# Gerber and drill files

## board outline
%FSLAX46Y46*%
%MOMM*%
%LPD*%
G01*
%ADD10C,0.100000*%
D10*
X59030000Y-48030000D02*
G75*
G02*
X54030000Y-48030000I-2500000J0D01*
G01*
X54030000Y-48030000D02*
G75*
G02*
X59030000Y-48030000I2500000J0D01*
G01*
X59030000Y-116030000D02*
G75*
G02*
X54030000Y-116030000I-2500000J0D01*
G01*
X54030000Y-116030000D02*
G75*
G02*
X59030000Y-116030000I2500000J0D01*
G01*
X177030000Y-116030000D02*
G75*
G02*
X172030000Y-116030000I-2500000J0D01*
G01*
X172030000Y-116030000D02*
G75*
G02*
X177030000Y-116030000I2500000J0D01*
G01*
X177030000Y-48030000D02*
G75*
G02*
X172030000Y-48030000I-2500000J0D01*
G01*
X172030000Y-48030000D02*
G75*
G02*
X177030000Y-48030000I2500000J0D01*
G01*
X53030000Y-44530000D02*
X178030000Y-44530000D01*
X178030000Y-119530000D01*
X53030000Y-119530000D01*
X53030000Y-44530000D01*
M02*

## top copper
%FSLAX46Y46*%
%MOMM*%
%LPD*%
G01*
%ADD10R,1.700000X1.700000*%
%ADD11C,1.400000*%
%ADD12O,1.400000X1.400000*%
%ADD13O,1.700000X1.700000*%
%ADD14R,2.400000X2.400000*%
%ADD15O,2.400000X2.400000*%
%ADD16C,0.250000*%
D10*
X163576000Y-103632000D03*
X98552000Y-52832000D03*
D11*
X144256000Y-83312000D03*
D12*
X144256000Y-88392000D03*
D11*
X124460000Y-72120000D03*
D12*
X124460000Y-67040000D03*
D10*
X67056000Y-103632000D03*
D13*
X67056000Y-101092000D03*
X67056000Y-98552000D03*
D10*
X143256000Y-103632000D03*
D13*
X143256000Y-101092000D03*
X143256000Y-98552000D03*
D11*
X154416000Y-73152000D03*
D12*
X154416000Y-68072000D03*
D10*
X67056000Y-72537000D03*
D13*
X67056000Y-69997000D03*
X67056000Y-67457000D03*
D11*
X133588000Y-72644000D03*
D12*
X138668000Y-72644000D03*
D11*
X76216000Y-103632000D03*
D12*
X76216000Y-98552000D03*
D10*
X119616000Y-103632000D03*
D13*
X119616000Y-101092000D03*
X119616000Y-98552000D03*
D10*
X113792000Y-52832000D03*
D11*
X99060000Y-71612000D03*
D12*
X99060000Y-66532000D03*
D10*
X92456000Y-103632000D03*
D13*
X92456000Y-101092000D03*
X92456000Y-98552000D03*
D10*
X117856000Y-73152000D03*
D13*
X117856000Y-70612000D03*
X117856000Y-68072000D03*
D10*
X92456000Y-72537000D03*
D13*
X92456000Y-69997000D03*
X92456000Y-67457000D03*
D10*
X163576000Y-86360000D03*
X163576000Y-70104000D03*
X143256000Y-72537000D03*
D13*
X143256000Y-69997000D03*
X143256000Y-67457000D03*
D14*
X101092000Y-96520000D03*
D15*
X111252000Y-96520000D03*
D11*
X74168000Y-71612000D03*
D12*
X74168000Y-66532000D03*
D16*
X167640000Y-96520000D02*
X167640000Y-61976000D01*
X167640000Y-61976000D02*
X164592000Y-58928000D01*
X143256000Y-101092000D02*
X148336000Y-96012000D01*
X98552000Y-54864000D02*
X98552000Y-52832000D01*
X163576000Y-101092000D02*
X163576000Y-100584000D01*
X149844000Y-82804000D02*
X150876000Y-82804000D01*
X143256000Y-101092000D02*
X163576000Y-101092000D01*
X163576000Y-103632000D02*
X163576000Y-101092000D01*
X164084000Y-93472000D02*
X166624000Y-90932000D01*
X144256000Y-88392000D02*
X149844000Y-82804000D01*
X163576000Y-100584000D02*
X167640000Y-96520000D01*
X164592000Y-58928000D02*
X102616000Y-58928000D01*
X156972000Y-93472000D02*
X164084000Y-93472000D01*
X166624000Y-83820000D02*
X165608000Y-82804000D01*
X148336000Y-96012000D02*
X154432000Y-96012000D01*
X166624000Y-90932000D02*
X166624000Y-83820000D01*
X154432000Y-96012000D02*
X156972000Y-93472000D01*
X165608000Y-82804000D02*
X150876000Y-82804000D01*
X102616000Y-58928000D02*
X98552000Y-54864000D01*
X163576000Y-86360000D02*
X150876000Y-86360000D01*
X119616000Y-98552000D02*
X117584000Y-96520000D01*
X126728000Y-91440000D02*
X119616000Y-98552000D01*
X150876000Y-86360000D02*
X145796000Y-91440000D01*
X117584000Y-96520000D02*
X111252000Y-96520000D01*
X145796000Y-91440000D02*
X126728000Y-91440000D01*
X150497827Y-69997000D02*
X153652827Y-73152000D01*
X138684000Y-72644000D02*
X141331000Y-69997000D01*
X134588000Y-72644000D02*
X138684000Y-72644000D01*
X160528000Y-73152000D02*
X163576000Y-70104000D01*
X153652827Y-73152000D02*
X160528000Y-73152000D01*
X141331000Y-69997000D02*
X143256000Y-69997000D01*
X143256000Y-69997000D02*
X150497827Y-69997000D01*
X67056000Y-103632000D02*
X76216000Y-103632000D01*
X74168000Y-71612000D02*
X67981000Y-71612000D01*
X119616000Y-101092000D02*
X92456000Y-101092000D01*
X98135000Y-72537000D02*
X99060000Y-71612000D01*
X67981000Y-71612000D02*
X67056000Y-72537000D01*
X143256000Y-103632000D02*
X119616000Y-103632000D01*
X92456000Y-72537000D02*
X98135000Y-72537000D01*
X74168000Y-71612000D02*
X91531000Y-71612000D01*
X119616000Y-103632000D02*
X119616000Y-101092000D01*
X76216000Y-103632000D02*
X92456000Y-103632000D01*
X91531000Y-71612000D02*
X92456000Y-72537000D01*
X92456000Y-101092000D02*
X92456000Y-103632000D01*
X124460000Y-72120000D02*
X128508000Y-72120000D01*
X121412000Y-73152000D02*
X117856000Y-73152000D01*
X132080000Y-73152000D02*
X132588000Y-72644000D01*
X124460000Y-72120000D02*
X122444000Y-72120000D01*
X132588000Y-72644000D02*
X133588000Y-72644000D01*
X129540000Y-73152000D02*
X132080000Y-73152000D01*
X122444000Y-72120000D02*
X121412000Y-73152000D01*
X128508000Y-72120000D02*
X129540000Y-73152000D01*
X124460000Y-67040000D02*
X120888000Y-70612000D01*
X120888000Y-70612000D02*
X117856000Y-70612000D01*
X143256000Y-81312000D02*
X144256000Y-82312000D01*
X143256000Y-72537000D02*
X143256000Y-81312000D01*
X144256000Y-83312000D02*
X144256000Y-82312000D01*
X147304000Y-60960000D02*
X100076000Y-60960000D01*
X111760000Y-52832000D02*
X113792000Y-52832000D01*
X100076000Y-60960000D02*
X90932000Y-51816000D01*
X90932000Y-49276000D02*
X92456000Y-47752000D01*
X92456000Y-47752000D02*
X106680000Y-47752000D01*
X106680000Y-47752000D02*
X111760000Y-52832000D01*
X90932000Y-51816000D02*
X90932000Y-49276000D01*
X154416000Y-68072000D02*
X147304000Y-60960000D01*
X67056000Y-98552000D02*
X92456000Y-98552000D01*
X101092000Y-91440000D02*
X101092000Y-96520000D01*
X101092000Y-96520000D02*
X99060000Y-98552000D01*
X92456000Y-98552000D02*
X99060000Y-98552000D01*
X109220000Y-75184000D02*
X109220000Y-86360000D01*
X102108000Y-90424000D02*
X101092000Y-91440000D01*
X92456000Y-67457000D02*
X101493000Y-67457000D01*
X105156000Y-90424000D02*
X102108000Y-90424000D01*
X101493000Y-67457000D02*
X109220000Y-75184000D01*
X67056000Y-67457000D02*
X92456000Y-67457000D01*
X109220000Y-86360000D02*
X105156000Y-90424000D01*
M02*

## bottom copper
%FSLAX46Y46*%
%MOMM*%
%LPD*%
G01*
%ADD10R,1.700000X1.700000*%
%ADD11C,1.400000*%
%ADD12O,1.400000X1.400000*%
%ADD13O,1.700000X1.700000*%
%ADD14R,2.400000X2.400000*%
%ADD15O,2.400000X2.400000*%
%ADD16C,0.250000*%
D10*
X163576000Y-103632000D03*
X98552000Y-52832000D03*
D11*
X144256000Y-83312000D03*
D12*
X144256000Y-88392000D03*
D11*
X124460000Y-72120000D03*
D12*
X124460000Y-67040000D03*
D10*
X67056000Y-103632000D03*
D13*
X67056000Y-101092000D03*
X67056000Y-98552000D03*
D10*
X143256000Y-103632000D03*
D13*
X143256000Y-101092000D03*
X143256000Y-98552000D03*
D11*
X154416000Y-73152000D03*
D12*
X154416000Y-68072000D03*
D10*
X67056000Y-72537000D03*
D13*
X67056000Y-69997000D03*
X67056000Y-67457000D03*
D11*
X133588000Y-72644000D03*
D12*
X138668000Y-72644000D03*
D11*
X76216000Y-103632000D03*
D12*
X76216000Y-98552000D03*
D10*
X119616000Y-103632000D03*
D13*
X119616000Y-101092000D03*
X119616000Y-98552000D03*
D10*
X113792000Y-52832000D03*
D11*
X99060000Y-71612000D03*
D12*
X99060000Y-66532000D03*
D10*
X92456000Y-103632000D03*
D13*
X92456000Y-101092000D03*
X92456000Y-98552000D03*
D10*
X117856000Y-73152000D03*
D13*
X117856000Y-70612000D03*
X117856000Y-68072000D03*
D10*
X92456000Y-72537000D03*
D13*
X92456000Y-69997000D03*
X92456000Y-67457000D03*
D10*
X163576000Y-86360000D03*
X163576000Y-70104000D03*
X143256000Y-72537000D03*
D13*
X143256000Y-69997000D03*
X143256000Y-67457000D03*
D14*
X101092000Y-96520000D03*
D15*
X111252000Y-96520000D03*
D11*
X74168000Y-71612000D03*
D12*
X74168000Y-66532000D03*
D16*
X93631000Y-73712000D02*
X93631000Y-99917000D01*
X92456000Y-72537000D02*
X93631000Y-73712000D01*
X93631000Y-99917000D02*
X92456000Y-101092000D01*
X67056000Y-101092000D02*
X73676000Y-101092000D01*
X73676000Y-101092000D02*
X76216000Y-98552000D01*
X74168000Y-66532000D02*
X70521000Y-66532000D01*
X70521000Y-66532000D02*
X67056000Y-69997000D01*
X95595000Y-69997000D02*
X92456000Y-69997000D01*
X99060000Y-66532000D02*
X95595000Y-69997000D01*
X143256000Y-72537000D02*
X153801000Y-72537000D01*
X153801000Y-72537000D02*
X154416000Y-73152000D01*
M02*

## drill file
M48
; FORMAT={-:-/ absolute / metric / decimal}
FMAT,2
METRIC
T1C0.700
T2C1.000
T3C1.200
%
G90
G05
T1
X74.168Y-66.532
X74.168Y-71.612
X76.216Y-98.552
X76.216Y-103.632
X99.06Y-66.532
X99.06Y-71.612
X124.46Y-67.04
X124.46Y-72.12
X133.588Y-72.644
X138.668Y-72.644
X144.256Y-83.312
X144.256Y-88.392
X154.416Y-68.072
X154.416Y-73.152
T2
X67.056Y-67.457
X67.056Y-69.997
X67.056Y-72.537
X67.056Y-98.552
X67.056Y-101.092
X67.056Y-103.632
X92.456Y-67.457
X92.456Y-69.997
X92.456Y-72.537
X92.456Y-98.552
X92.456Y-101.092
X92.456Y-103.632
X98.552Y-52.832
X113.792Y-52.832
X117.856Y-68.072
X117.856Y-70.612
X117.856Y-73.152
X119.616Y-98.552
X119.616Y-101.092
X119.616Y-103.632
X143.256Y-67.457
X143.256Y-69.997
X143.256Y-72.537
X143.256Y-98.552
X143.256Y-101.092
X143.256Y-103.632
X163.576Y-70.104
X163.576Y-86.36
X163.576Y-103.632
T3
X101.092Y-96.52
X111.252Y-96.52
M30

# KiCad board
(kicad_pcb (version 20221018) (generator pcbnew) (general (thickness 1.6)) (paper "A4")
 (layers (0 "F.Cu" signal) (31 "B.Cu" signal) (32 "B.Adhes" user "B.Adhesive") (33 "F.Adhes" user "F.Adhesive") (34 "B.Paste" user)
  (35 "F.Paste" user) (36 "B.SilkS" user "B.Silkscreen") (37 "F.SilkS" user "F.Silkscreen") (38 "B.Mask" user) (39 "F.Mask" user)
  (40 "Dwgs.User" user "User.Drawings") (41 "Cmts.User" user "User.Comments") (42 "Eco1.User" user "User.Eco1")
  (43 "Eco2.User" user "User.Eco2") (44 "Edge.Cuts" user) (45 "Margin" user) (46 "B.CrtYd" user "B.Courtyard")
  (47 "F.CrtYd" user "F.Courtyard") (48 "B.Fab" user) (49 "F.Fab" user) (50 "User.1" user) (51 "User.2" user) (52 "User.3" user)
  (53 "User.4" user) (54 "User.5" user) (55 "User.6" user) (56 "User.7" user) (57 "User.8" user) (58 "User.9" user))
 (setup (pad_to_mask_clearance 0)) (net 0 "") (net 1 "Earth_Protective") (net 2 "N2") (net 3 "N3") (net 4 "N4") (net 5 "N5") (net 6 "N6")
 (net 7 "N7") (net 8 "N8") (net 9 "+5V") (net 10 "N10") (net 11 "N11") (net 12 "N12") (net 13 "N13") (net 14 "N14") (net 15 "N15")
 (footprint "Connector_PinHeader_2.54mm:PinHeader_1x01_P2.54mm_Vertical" (layer "F.Cu") (at 163.576 103.632 180)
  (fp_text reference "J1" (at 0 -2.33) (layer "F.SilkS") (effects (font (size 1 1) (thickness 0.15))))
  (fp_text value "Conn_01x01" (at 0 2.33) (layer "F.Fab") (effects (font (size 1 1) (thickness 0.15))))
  (pad "1" thru_hole rect (at 0 0 180) (size 1.7 1.7) (drill 1) (layers "*.Cu" "*.Mask") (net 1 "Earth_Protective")))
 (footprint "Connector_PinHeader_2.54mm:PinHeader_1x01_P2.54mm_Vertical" (layer "F.Cu") (at 98.552 52.832 180)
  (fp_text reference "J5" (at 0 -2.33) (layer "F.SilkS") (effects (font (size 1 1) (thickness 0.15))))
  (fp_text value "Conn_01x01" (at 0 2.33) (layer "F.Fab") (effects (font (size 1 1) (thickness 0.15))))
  (pad "1" thru_hole rect (at 0 0 180) (size 1.7 1.7) (drill 1) (layers "*.Cu" "*.Mask") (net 1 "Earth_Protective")))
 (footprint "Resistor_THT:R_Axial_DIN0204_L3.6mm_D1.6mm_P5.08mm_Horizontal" (layer "F.Cu") (at 144.256 83.312 -90)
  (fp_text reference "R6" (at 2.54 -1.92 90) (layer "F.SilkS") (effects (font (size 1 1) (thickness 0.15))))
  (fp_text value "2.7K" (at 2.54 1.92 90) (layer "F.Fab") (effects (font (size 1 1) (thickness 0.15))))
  (pad "1" thru_hole circle (at 0 0 270) (size 1.4 1.4) (drill 0.7) (layers "*.Cu" "*.Mask") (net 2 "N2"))
  (pad "2" thru_hole oval (at 5.08 0 270) (size 1.4 1.4) (drill 0.7) (layers "*.Cu" "*.Mask") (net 1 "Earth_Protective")))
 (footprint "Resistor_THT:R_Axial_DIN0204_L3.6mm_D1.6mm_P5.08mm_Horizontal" (layer "F.Cu") (at 124.46 72.12 90)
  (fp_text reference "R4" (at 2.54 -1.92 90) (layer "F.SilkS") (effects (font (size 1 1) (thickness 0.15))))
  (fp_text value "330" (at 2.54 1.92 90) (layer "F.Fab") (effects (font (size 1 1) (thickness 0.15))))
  (pad "1" thru_hole circle (at 0 0 90) (size 1.4 1.4) (drill 0.7) (layers "*.Cu" "*.Mask") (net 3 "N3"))
  (pad "2" thru_hole oval (at 5.08 0 90) (size 1.4 1.4) (drill 0.7) (layers "*.Cu" "*.Mask") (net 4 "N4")))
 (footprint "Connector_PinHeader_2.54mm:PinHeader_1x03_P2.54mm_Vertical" (layer "F.Cu") (at 67.056 103.632 180)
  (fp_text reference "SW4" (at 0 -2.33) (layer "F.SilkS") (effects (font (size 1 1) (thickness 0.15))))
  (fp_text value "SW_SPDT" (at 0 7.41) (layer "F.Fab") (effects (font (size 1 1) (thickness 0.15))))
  (pad "1" thru_hole rect (at 0 0 180) (size 1.7 1.7) (drill 1) (layers "*.Cu" "*.Mask") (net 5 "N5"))
  (pad "2" thru_hole oval (at 0 2.54 180) (size 1.7 1.7) (drill 1) (layers "*.Cu" "*.Mask") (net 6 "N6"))
  (pad "3" thru_hole oval (at 0 5.08 180) (size 1.7 1.7) (drill 1) (layers "*.Cu" "*.Mask") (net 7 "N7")))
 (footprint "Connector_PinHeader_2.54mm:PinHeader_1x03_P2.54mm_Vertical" (layer "F.Cu") (at 143.256 103.632 180)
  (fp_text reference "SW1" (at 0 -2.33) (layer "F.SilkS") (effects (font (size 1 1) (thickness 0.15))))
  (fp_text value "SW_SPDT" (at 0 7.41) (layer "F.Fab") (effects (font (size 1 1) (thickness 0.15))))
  (pad "1" thru_hole rect (at 0 0 180) (size 1.7 1.7) (drill 1) (layers "*.Cu" "*.Mask") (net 5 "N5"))
  (pad "2" thru_hole oval (at 0 2.54 180) (size 1.7 1.7) (drill 1) (layers "*.Cu" "*.Mask") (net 1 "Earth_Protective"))
  (pad "3" thru_hole oval (at 0 5.08 180) (size 1.7 1.7) (drill 1) (layers "*.Cu" "*.Mask") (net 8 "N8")))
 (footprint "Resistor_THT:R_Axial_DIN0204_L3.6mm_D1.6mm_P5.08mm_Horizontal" (layer "F.Cu") (at 154.416 73.152 90)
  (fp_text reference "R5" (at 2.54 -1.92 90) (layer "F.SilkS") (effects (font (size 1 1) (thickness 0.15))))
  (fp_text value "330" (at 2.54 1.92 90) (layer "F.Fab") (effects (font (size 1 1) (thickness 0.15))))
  (pad "1" thru_hole circle (at 0 0 90) (size 1.4 1.4) (drill 0.7) (layers "*.Cu" "*.Mask") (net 2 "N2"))
  (pad "2" thru_hole oval (at 5.08 0 90) (size 1.4 1.4) (drill 0.7) (layers "*.Cu" "*.Mask") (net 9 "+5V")))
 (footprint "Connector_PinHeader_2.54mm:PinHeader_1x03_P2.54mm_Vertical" (layer "F.Cu") (at 67.056 72.537 180)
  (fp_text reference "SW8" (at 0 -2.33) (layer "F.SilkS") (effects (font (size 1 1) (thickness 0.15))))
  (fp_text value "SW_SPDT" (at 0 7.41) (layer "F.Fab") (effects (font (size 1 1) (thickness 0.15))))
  (pad "1" thru_hole rect (at 0 0 180) (size 1.7 1.7) (drill 1) (layers "*.Cu" "*.Mask") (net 5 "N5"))
  (pad "2" thru_hole oval (at 0 2.54 180) (size 1.7 1.7) (drill 1) (layers "*.Cu" "*.Mask") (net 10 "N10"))
  (pad "3" thru_hole oval (at 0 5.08 180) (size 1.7 1.7) (drill 1) (layers "*.Cu" "*.Mask") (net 7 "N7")))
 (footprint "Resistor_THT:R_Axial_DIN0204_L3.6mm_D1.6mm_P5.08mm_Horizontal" (layer "F.Cu") (at 133.588 72.644)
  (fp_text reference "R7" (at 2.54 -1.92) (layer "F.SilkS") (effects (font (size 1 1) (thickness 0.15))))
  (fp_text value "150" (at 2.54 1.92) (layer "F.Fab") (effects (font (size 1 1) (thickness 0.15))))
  (pad "1" thru_hole circle (at 0 0) (size 1.4 1.4) (drill 0.7) (layers "*.Cu" "*.Mask") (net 3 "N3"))
  (pad "2" thru_hole oval (at 5.08 0) (size 1.4 1.4) (drill 0.7) (layers "*.Cu" "*.Mask") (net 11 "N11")))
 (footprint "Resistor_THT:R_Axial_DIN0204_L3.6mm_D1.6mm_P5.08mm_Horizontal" (layer "F.Cu") (at 76.216 103.632 90)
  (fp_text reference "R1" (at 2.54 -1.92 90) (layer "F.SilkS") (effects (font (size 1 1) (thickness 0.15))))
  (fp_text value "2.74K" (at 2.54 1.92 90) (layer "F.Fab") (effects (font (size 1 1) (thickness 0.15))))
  (pad "1" thru_hole circle (at 0 0 90) (size 1.4 1.4) (drill 0.7) (layers "*.Cu" "*.Mask") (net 5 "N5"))
  (pad "2" thru_hole oval (at 5.08 0 90) (size 1.4 1.4) (drill 0.7) (layers "*.Cu" "*.Mask") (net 6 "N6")))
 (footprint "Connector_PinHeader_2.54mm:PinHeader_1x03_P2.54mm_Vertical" (layer "F.Cu") (at 119.616 103.632 180)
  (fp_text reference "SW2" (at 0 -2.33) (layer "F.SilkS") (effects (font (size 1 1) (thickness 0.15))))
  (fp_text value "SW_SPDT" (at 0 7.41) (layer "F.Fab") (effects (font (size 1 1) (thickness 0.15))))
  (pad "1" thru_hole rect (at 0 0 180) (size 1.7 1.7) (drill 1) (layers "*.Cu" "*.Mask") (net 5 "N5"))
  (pad "2" thru_hole oval (at 0 2.54 180) (size 1.7 1.7) (drill 1) (layers "*.Cu" "*.Mask") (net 5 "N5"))
  (pad "3" thru_hole oval (at 0 5.08 180) (size 1.7 1.7) (drill 1) (layers "*.Cu" "*.Mask") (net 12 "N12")))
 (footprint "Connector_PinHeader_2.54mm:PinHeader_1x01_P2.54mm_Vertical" (layer "F.Cu") (at 113.792 52.832 180)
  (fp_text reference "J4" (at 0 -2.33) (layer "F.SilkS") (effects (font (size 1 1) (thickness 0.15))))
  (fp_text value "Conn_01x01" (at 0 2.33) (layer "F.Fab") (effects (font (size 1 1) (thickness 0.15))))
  (pad "1" thru_hole rect (at 0 0 180) (size 1.7 1.7) (drill 1) (layers "*.Cu" "*.Mask") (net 9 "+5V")))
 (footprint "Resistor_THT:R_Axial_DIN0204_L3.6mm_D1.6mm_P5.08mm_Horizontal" (layer "F.Cu") (at 99.06 71.612 90)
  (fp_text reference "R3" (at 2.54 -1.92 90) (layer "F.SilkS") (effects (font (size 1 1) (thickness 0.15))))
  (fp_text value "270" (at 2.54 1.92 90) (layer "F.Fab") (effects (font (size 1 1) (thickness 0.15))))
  (pad "1" thru_hole circle (at 0 0 90) (size 1.4 1.4) (drill 0.7) (layers "*.Cu" "*.Mask") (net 5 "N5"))
  (pad "2" thru_hole oval (at 5.08 0 90) (size 1.4 1.4) (drill 0.7) (layers "*.Cu" "*.Mask") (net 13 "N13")))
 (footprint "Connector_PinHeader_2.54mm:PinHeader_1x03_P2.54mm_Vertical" (layer "F.Cu") (at 92.456 103.632 180)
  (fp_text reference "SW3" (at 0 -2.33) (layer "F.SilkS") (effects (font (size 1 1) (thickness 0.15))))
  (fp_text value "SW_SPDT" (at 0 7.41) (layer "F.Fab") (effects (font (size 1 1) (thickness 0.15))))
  (pad "1" thru_hole rect (at 0 0 180) (size 1.7 1.7) (drill 1) (layers "*.Cu" "*.Mask") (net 5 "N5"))
  (pad "2" thru_hole oval (at 0 2.54 180) (size 1.7 1.7) (drill 1) (layers "*.Cu" "*.Mask") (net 5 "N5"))
  (pad "3" thru_hole oval (at 0 5.08 180) (size 1.7 1.7) (drill 1) (layers "*.Cu" "*.Mask") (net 7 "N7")))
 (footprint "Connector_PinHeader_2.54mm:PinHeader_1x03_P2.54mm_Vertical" (layer "F.Cu") (at 117.856 73.152 180)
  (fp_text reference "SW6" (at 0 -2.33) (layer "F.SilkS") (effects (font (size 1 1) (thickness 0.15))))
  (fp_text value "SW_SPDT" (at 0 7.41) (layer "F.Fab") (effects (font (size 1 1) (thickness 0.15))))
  (pad "1" thru_hole rect (at 0 0 180) (size 1.7 1.7) (drill 1) (layers "*.Cu" "*.Mask") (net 3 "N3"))
  (pad "2" thru_hole oval (at 0 2.54 180) (size 1.7 1.7) (drill 1) (layers "*.Cu" "*.Mask") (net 4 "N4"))
  (pad "3" thru_hole oval (at 0 5.08 180) (size 1.7 1.7) (drill 1) (layers "*.Cu" "*.Mask") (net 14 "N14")))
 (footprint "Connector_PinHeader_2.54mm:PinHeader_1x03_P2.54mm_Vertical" (layer "F.Cu") (at 92.456 72.537 180)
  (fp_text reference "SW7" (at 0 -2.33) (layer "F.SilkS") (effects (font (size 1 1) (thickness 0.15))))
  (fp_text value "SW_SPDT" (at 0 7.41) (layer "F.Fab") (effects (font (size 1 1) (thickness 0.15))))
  (pad "1" thru_hole rect (at 0 0 180) (size 1.7 1.7) (drill 1) (layers "*.Cu" "*.Mask") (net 5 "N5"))
  (pad "2" thru_hole oval (at 0 2.54 180) (size 1.7 1.7) (drill 1) (layers "*.Cu" "*.Mask") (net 13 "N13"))
  (pad "3" thru_hole oval (at 0 5.08 180) (size 1.7 1.7) (drill 1) (layers "*.Cu" "*.Mask") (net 7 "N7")))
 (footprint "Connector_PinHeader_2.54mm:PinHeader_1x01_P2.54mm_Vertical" (layer "F.Cu") (at 163.576 86.36 180)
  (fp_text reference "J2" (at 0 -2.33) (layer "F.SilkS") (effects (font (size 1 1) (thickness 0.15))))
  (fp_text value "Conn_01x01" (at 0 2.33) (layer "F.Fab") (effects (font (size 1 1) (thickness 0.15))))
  (pad "1" thru_hole rect (at 0 0 180) (size 1.7 1.7) (drill 1) (layers "*.Cu" "*.Mask") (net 12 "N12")))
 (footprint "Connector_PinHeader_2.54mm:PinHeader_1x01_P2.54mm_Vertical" (layer "F.Cu") (at 163.576 70.104 180)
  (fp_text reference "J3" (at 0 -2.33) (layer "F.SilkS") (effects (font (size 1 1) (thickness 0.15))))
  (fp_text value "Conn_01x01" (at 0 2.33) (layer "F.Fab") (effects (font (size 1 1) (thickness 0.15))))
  (pad "1" thru_hole rect (at 0 0 180) (size 1.7 1.7) (drill 1) (layers "*.Cu" "*.Mask") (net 11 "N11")))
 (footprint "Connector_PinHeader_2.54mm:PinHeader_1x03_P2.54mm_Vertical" (layer "F.Cu") (at 143.256 72.537 180)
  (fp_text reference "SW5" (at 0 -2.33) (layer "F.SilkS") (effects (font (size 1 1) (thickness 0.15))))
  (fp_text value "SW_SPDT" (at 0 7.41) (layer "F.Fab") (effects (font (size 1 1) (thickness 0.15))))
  (pad "1" thru_hole rect (at 0 0 180) (size 1.7 1.7) (drill 1) (layers "*.Cu" "*.Mask") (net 2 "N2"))
  (pad "2" thru_hole oval (at 0 2.54 180) (size 1.7 1.7) (drill 1) (layers "*.Cu" "*.Mask") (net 11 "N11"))
  (pad "3" thru_hole oval (at 0 5.08 180) (size 1.7 1.7) (drill 1) (layers "*.Cu" "*.Mask") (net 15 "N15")))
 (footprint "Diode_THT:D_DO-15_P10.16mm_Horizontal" (layer "F.Cu") (at 101.092 96.52)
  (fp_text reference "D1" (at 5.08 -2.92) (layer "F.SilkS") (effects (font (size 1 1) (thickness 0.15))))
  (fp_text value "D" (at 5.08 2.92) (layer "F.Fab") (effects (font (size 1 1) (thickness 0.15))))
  (pad "1" thru_hole rect (at 0 0) (size 2.4 2.4) (drill 1.2) (layers "*.Cu" "*.Mask") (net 7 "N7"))
  (pad "2" thru_hole oval (at 10.16 0) (size 2.4 2.4) (drill 1.2) (layers "*.Cu" "*.Mask") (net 12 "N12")))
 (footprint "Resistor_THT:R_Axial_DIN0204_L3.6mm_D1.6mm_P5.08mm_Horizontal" (layer "F.Cu") (at 74.168 71.612 90)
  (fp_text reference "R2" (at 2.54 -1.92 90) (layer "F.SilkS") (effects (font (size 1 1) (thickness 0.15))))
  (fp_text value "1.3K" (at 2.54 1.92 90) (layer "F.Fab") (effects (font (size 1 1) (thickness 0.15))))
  (pad "1" thru_hole circle (at 0 0 90) (size 1.4 1.4) (drill 0.7) (layers "*.Cu" "*.Mask") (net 5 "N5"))
  (pad "2" thru_hole oval (at 5.08 0 90) (size 1.4 1.4) (drill 0.7) (layers "*.Cu" "*.Mask") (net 10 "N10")))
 (gr_circle (center 56.53 48.03) (end 54.03 48.03) (stroke (width 0.1) (type default)) (fill none) (layer "Edge.Cuts"))
 (gr_circle (center 56.53 116.03) (end 54.03 116.03) (stroke (width 0.1) (type default)) (fill none) (layer "Edge.Cuts"))
 (gr_circle (center 174.53 116.03) (end 172.03 116.03) (stroke (width 0.1) (type default)) (fill none) (layer "Edge.Cuts"))
 (gr_circle (center 174.53 48.03) (end 172.03 48.03) (stroke (width 0.1) (type default)) (fill none) (layer "Edge.Cuts"))
 (gr_rect (start 178.03 119.53) (end 53.03 44.53) (stroke (width 0.1) (type default)) (fill none) (layer "Edge.Cuts"))
 (segment (start 167.64 96.52) (end 167.64 61.976) (width 0.25) (layer "F.Cu") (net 1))
 (segment (start 167.64 61.976) (end 164.592 58.928) (width 0.25) (layer "F.Cu") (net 1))
 (segment (start 143.256 101.092) (end 148.336 96.012) (width 0.25) (layer "F.Cu") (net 1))
 (segment (start 98.552 54.864) (end 98.552 52.832) (width 0.25) (layer "F.Cu") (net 1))
 (segment (start 163.576 101.092) (end 163.576 100.584) (width 0.25) (layer "F.Cu") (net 1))
 (segment (start 149.844 82.804) (end 150.876 82.804) (width 0.25) (layer "F.Cu") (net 1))
 (segment (start 143.256 101.092) (end 163.576 101.092) (width 0.25) (layer "F.Cu") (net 1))
 (segment (start 163.576 103.632) (end 163.576 101.092) (width 0.25) (layer "F.Cu") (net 1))
 (segment (start 164.084 93.472) (end 166.624 90.932) (width 0.25) (layer "F.Cu") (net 1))
 (segment (start 144.256 88.392) (end 149.844 82.804) (width 0.25) (layer "F.Cu") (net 1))
 (segment (start 163.576 100.584) (end 167.64 96.52) (width 0.25) (layer "F.Cu") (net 1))
 (segment (start 164.592 58.928) (end 102.616 58.928) (width 0.25) (layer "F.Cu") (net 1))
 (segment (start 156.972 93.472) (end 164.084 93.472) (width 0.25) (layer "F.Cu") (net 1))
 (segment (start 166.624 83.82) (end 165.608 82.804) (width 0.25) (layer "F.Cu") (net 1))
 (segment (start 148.336 96.012) (end 154.432 96.012) (width 0.25) (layer "F.Cu") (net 1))
 (segment (start 166.624 90.932) (end 166.624 83.82) (width 0.25) (layer "F.Cu") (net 1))
 (segment (start 154.432 96.012) (end 156.972 93.472) (width 0.25) (layer "F.Cu") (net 1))
 (segment (start 165.608 82.804) (end 150.876 82.804) (width 0.25) (layer "F.Cu") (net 1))
 (segment (start 102.616 58.928) (end 98.552 54.864) (width 0.25) (layer "F.Cu") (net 1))
 (segment (start 163.576 86.36) (end 150.876 86.36) (width 0.25) (layer "F.Cu") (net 12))
 (segment (start 119.616 98.552) (end 117.584 96.52) (width 0.25) (layer "F.Cu") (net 12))
 (segment (start 126.728 91.44) (end 119.616 98.552) (width 0.25) (layer "F.Cu") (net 12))
 (segment (start 150.876 86.36) (end 145.796 91.44) (width 0.25) (layer "F.Cu") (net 12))
 (segment (start 117.584 96.52) (end 111.252 96.52) (width 0.25) (layer "F.Cu") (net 12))
 (segment (start 145.796 91.44) (end 126.728 91.44) (width 0.25) (layer "F.Cu") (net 12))
 (segment (start 150.497827 69.997) (end 153.652827 73.152) (width 0.25) (layer "F.Cu") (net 11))
 (segment (start 138.684 72.644) (end 141.331 69.997) (width 0.25) (layer "F.Cu") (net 11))
 (segment (start 134.588 72.644) (end 138.684 72.644) (width 0.25) (layer "F.Cu") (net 11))
 (segment (start 160.528 73.152) (end 163.576 70.104) (width 0.25) (layer "F.Cu") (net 11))
 (segment (start 153.652827 73.152) (end 160.528 73.152) (width 0.25) (layer "F.Cu") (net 11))
 (segment (start 141.331 69.997) (end 143.256 69.997) (width 0.25) (layer "F.Cu") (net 11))
 (segment (start 143.256 69.997) (end 150.497827 69.997) (width 0.25) (layer "F.Cu") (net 11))
 (segment (start 67.056 103.632) (end 76.216 103.632) (width 0.25) (layer "F.Cu") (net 5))
 (segment (start 74.168 71.612) (end 67.981 71.612) (width 0.25) (layer "F.Cu") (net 5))
 (segment (start 119.616 101.092) (end 92.456 101.092) (width 0.25) (layer "F.Cu") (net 5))
 (segment (start 98.135 72.537) (end 99.06 71.612) (width 0.25) (layer "F.Cu") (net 5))
 (segment (start 67.981 71.612) (end 67.056 72.537) (width 0.25) (layer "F.Cu") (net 5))
 (segment (start 143.256 103.632) (end 119.616 103.632) (width 0.25) (layer "F.Cu") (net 5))
 (segment (start 92.456 72.537) (end 98.135 72.537) (width 0.25) (layer "F.Cu") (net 5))
 (segment (start 74.168 71.612) (end 91.531 71.612) (width 0.25) (layer "F.Cu") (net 5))
 (segment (start 119.616 103.632) (end 119.616 101.092) (width 0.25) (layer "F.Cu") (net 5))
 (segment (start 76.216 103.632) (end 92.456 103.632) (width 0.25) (layer "F.Cu") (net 5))
 (segment (start 91.531 71.612) (end 92.456 72.537) (width 0.25) (layer "F.Cu") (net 5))
 (segment (start 92.456 101.092) (end 92.456 103.632) (width 0.25) (layer "F.Cu") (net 5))
 (segment (start 93.631 73.712) (end 93.631 99.917) (width 0.25) (layer "B.Cu") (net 5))
 (segment (start 92.456 72.537) (end 93.631 73.712) (width 0.25) (layer "B.Cu") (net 5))
 (segment (start 93.631 99.917) (end 92.456 101.092) (width 0.25) (layer "B.Cu") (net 5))
 (segment (start 67.056 101.092) (end 73.676 101.092) (width 0.25) (layer "B.Cu") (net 6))
 (segment (start 73.676 101.092) (end 76.216 98.552) (width 0.25) (layer "B.Cu") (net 6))
 (segment (start 74.168 66.532) (end 70.521 66.532) (width 0.25) (layer "B.Cu") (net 10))
 (segment (start 70.521 66.532) (end 67.056 69.997) (width 0.25) (layer "B.Cu") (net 10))
 (segment (start 95.595 69.997) (end 92.456 69.997) (width 0.25) (layer "B.Cu") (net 13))
 (segment (start 99.06 66.532) (end 95.595 69.997) (width 0.25) (layer "B.Cu") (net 13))
 (segment (start 124.46 72.12) (end 128.508 72.12) (width 0.25) (layer "F.Cu") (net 3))
 (segment (start 121.412 73.152) (end 117.856 73.152) (width 0.25) (layer "F.Cu") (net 3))
 (segment (start 132.08 73.152) (end 132.588 72.644) (width 0.25) (layer "F.Cu") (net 3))
 (segment (start 124.46 72.12) (end 122.444 72.12) (width 0.25) (layer "F.Cu") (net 3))
 (segment (start 132.588 72.644) (end 133.588 72.644) (width 0.25) (layer "F.Cu") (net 3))
 (segment (start 129.54 73.152) (end 132.08 73.152) (width 0.25) (layer "F.Cu") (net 3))
 (segment (start 122.444 72.12) (end 121.412 73.152) (width 0.25) (layer "F.Cu") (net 3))
 (segment (start 128.508 72.12) (end 129.54 73.152) (width 0.25) (layer "F.Cu") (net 3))
 (segment (start 124.46 67.04) (end 120.888 70.612) (width 0.25) (layer "F.Cu") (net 4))
 (segment (start 120.888 70.612) (end 117.856 70.612) (width 0.25) (layer "F.Cu") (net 4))
 (segment (start 143.256 81.312) (end 144.256 82.312) (width 0.25) (layer "F.Cu") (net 2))
 (segment (start 143.256 72.537) (end 143.256 81.312) (width 0.25) (layer "F.Cu") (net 2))
 (segment (start 144.256 83.312) (end 144.256 82.312) (width 0.25) (layer "F.Cu") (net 2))
 (segment (start 143.256 72.537) (end 153.801 72.537) (width 0.25) (layer "B.Cu") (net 2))
 (segment (start 153.801 72.537) (end 154.416 73.152) (width 0.25) (layer "B.Cu") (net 2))
 (segment (start 147.304 60.96) (end 100.076 60.96) (width 0.25) (layer "F.Cu") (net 9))
 (segment (start 111.76 52.832) (end 113.792 52.832) (width 0.25) (layer "F.Cu") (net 9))
 (segment (start 100.076 60.96) (end 90.932 51.816) (width 0.25) (layer "F.Cu") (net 9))
 (segment (start 90.932 49.276) (end 92.456 47.752) (width 0.25) (layer "F.Cu") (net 9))
 (segment (start 92.456 47.752) (end 106.68 47.752) (width 0.25) (layer "F.Cu") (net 9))
 (segment (start 106.68 47.752) (end 111.76 52.832) (width 0.25) (layer "F.Cu") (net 9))
 (segment (start 90.932 51.816) (end 90.932 49.276) (width 0.25) (layer "F.Cu") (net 9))
 (segment (start 154.416 68.072) (end 147.304 60.96) (width 0.25) (layer "F.Cu") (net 9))
 (segment (start 67.056 98.552) (end 92.456 98.552) (width 0.25) (layer "F.Cu") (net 7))
 (segment (start 101.092 91.44) (end 101.092 96.52) (width 0.25) (layer "F.Cu") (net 7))
 (segment (start 101.092 96.52) (end 99.06 98.552) (width 0.25) (layer "F.Cu") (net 7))
 (segment (start 92.456 98.552) (end 99.06 98.552) (width 0.25) (layer "F.Cu") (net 7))
 (segment (start 109.22 75.184) (end 109.22 86.36) (width 0.25) (layer "F.Cu") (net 7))
 (segment (start 102.108 90.424) (end 101.092 91.44) (width 0.25) (layer "F.Cu") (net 7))
 (segment (start 92.456 67.457) (end 101.493 67.457) (width 0.25) (layer "F.Cu") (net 7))
 (segment (start 105.156 90.424) (end 102.108 90.424) (width 0.25) (layer "F.Cu") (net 7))
 (segment (start 101.493 67.457) (end 109.22 75.184) (width 0.25) (layer "F.Cu") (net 7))
 (segment (start 67.056 67.457) (end 92.456 67.457) (width 0.25) (layer "F.Cu") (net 7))
 (segment (start 109.22 86.36) (end 105.156 90.424) (width 0.25) (layer "F.Cu") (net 7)))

